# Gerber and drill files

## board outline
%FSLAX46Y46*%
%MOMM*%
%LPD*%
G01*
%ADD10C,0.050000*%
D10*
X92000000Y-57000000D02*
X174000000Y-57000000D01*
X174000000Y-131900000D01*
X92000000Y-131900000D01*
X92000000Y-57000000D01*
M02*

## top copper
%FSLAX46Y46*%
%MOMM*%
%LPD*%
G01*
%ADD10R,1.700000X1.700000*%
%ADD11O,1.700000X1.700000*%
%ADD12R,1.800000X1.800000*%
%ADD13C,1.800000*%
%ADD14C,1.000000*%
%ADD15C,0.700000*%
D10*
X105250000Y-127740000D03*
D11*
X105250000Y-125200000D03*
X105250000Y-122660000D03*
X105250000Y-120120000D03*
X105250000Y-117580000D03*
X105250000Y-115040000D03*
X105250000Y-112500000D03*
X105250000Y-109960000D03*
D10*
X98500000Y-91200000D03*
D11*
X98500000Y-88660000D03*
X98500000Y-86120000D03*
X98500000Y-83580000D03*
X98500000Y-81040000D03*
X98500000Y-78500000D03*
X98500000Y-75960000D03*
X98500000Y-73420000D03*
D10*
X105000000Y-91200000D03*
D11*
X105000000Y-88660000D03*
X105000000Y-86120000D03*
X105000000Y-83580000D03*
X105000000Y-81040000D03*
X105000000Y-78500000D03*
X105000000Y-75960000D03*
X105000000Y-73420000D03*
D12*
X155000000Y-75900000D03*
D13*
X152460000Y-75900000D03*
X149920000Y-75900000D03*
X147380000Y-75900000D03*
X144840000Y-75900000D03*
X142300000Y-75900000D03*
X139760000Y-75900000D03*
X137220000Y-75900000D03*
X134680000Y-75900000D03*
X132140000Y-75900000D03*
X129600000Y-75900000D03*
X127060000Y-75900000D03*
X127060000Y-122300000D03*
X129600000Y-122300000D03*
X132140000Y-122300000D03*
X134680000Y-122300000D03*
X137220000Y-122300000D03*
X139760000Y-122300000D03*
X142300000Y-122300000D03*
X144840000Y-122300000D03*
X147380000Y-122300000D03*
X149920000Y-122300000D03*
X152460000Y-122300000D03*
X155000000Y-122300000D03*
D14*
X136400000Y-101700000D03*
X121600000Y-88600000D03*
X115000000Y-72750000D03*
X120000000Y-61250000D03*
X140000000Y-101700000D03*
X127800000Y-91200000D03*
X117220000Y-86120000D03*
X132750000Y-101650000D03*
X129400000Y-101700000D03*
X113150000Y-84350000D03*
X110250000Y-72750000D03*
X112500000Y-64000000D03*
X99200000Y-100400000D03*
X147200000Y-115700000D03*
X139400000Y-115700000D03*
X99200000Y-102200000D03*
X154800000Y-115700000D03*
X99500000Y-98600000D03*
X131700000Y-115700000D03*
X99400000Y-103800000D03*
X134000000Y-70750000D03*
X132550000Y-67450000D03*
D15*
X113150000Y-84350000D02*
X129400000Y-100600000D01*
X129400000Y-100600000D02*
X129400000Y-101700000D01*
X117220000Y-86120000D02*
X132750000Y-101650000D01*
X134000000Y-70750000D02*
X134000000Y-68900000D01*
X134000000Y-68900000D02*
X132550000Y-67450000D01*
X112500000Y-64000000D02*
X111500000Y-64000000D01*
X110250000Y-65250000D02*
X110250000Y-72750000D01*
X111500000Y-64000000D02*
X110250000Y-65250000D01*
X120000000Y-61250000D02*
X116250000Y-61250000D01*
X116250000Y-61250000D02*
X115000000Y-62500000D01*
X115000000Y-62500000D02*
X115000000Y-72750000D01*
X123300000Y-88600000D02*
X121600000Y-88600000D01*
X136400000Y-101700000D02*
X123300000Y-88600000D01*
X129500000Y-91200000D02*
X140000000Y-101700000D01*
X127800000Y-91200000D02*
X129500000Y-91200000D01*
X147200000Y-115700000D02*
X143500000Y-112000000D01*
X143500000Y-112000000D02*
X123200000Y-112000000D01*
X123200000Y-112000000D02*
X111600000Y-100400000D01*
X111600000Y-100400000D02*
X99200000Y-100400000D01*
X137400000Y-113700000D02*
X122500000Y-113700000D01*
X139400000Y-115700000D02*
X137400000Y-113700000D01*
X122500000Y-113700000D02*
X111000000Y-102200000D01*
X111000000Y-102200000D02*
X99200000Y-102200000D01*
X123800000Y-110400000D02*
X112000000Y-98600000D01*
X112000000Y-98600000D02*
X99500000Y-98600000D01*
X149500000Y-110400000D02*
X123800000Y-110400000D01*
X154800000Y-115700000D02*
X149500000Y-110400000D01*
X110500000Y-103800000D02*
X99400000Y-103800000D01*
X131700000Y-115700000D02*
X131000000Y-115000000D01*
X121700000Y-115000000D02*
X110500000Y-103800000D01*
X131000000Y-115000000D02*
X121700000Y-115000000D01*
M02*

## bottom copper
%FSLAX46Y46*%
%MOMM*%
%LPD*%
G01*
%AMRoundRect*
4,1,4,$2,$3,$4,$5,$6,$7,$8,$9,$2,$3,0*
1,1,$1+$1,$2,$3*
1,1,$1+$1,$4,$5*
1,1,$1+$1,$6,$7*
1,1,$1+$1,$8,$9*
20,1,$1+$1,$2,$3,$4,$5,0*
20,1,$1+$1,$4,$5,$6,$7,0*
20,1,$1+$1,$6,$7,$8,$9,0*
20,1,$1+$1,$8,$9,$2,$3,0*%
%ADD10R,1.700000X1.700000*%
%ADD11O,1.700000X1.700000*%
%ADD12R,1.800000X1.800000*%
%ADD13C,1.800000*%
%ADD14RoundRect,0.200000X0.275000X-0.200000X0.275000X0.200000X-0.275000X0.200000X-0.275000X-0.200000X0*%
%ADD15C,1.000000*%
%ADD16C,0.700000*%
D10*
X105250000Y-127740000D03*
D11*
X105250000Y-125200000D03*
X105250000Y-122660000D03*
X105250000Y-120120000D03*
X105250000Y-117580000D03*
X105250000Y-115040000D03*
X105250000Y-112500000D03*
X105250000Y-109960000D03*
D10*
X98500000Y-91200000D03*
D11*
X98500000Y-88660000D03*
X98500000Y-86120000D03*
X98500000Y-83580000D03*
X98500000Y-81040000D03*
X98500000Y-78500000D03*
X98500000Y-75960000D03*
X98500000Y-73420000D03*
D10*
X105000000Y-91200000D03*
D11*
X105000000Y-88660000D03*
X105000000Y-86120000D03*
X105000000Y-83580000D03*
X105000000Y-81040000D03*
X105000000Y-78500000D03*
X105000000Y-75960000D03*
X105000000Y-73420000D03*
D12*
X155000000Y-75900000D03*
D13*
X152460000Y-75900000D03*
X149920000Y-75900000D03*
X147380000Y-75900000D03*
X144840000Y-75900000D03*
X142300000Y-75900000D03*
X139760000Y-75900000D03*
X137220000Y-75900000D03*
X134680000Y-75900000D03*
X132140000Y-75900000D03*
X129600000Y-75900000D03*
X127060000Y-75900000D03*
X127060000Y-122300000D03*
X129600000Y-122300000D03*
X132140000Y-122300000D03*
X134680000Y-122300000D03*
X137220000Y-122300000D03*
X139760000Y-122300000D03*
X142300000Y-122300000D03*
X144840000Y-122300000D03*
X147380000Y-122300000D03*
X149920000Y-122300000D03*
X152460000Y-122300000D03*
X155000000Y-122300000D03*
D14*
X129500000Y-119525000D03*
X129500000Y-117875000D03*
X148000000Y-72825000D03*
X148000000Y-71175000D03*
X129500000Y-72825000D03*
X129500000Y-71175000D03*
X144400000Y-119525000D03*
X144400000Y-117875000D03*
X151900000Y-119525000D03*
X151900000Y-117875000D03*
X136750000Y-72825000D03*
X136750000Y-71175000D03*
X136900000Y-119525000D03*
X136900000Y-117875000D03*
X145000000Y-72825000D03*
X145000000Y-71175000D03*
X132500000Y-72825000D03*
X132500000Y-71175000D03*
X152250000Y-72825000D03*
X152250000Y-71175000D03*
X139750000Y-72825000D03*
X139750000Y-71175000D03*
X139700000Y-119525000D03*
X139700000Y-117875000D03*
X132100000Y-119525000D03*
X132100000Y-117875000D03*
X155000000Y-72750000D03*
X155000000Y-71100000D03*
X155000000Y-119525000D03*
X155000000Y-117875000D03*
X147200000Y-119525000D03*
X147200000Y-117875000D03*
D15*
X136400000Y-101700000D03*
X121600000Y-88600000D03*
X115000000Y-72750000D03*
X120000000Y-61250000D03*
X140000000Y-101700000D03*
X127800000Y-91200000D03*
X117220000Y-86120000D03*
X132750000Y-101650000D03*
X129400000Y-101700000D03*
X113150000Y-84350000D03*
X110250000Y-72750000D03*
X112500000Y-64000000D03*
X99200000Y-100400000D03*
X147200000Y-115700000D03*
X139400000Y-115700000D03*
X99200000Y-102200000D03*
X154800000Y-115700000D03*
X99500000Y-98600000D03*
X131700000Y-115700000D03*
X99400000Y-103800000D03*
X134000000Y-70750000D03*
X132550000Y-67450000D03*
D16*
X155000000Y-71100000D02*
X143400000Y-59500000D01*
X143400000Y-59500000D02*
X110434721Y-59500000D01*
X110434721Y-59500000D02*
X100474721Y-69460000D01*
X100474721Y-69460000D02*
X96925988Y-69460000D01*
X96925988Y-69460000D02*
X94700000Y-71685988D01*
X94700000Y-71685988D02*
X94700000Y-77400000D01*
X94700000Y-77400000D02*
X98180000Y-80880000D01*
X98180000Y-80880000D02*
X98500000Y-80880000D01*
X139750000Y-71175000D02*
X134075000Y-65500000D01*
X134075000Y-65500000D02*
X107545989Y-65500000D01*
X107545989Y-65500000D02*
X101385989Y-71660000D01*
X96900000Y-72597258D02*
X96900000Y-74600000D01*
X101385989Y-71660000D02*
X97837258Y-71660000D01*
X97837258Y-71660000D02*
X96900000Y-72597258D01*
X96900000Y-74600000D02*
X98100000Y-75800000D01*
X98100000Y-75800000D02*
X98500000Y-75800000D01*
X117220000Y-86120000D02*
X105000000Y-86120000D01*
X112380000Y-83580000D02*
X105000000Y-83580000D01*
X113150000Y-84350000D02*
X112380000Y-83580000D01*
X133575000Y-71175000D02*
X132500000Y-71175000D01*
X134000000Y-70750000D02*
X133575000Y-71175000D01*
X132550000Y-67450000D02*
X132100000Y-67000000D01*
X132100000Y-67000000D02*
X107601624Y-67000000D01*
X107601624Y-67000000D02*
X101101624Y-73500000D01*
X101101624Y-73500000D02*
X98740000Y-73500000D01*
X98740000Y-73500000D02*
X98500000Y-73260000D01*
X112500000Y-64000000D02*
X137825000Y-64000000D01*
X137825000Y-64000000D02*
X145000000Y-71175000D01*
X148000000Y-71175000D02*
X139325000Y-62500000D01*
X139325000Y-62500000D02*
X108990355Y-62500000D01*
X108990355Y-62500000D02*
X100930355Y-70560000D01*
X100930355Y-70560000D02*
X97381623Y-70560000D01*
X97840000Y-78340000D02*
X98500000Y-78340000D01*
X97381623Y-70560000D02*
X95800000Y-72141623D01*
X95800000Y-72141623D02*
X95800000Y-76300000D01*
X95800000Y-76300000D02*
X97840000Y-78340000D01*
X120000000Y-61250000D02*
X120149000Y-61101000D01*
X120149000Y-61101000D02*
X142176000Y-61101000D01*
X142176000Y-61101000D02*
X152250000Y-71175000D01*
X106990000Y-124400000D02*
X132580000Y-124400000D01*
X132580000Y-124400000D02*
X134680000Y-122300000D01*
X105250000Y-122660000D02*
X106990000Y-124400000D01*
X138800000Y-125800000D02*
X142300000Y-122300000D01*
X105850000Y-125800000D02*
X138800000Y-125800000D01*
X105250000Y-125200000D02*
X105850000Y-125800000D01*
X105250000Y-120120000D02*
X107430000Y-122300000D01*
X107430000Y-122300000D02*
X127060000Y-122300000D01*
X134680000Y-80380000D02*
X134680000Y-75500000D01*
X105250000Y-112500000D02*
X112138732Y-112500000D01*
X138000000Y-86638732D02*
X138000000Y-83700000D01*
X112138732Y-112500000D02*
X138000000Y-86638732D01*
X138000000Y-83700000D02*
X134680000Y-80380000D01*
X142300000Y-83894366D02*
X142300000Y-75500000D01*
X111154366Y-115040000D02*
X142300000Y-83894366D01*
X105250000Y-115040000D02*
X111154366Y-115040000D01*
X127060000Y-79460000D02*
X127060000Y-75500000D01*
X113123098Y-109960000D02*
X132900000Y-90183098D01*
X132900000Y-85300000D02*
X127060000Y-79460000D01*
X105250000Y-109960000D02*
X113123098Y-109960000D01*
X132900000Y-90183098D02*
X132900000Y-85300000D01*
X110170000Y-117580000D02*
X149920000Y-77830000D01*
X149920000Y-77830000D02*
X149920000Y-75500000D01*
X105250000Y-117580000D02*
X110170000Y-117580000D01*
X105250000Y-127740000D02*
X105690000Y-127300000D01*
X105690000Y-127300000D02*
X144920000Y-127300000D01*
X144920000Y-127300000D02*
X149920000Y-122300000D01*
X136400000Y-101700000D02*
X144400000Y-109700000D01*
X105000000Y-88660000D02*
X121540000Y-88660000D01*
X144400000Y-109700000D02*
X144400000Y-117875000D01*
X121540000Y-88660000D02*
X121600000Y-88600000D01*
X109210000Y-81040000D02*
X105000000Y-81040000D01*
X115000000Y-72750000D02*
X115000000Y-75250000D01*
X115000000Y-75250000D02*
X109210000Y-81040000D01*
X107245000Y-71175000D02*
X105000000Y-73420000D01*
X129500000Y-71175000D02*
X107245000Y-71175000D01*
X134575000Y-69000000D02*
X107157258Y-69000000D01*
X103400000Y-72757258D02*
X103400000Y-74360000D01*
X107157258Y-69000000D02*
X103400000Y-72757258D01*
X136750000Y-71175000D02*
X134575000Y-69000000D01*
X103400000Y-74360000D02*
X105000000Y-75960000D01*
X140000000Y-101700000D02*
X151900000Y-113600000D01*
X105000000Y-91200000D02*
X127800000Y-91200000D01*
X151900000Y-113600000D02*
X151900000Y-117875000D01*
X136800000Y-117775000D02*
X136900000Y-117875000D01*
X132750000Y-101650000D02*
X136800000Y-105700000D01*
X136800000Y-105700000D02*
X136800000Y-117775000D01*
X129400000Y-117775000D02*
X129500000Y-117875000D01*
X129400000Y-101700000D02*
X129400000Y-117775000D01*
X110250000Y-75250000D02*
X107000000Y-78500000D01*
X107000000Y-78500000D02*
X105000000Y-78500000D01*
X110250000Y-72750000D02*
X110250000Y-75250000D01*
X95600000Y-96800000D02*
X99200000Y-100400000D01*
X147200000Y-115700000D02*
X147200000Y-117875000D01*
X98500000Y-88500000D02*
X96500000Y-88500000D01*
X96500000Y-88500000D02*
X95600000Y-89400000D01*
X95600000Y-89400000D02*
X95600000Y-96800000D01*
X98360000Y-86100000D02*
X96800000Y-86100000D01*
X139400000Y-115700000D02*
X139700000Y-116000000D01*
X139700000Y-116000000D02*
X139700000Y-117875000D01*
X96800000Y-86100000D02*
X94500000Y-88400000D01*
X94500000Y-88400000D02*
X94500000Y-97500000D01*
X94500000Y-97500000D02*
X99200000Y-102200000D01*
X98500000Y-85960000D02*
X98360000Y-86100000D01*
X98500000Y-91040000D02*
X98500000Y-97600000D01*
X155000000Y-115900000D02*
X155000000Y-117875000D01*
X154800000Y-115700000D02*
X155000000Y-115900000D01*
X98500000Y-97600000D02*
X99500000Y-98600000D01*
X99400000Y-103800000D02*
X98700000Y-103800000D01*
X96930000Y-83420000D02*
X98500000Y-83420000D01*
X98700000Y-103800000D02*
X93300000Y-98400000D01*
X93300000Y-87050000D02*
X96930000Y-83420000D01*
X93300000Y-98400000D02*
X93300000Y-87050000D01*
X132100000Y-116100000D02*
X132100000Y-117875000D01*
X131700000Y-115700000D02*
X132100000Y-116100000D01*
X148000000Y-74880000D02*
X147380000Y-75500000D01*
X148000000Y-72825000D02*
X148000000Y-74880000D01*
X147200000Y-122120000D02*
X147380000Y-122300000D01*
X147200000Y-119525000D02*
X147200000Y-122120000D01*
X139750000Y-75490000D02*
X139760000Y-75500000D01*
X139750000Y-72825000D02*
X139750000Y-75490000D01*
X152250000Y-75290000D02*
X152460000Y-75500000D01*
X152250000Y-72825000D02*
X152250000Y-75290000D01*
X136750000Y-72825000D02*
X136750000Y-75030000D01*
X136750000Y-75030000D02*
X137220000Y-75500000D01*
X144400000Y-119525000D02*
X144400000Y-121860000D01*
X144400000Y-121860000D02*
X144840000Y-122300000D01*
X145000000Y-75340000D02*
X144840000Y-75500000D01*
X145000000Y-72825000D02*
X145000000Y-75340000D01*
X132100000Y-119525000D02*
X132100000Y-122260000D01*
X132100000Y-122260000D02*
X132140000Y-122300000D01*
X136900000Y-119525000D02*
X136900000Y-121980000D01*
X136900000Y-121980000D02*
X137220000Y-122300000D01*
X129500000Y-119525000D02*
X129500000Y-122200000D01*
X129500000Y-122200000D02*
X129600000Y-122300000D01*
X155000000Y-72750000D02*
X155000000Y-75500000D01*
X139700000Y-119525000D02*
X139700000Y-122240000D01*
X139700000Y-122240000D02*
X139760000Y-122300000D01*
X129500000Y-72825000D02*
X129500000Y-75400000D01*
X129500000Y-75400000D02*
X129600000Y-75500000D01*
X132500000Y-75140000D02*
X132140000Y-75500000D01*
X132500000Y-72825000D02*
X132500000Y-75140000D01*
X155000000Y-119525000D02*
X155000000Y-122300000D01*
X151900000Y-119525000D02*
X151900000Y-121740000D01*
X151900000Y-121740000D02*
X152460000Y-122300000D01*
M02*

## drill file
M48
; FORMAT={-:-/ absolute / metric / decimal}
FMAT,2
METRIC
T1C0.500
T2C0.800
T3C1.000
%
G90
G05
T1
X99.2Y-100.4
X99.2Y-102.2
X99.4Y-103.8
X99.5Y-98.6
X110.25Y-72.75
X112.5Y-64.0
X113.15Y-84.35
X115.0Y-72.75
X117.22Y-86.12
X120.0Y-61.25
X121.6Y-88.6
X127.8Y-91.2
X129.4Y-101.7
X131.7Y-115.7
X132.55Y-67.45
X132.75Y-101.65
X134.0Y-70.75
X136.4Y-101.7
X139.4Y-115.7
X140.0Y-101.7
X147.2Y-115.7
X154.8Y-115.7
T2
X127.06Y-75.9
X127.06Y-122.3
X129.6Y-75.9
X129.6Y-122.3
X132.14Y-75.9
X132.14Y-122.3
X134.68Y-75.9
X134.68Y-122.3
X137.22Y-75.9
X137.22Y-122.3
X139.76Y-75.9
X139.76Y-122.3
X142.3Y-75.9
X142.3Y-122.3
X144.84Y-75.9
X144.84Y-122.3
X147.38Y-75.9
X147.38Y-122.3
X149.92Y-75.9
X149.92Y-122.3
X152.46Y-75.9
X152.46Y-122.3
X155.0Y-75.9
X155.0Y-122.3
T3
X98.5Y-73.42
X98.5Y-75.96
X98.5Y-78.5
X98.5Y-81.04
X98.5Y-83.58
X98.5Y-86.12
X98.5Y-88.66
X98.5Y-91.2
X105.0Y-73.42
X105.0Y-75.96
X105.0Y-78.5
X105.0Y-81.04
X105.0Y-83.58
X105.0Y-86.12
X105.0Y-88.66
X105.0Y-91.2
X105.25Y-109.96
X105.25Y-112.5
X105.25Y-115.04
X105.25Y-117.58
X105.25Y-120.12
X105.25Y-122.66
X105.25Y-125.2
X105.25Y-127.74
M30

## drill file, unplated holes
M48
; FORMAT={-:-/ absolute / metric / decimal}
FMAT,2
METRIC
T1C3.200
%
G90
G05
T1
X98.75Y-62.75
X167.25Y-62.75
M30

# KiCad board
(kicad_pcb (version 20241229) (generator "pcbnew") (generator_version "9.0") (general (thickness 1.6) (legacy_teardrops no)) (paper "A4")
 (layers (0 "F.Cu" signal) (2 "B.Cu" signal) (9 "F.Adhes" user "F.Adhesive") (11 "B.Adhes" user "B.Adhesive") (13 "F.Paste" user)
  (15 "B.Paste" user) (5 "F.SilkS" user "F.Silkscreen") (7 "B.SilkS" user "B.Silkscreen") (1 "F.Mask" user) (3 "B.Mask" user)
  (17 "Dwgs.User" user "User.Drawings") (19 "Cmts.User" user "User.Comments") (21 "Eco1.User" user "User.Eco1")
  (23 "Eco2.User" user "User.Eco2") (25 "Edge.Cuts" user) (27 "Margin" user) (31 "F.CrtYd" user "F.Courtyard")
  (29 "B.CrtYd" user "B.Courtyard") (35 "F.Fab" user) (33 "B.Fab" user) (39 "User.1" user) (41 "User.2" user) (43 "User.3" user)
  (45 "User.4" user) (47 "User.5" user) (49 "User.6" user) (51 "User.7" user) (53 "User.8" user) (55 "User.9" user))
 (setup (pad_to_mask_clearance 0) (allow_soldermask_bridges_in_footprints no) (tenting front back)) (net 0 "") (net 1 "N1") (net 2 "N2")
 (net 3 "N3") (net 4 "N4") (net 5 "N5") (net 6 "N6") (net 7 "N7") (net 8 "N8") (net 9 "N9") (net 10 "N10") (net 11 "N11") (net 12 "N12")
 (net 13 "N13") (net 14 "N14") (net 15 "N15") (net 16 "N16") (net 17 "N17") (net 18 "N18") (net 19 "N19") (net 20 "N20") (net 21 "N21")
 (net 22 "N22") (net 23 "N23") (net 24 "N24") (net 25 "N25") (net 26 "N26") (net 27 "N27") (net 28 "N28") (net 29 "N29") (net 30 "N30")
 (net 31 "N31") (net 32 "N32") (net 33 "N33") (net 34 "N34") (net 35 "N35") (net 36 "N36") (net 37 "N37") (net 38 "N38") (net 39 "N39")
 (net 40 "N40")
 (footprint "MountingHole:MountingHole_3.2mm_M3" (layer "F.Cu") (at 98.75 62.75)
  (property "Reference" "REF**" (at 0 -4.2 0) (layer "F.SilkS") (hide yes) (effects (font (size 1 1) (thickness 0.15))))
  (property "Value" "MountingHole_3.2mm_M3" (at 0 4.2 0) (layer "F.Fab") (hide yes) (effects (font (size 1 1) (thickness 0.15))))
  (pad "" np_thru_hole circle (at 0 0) (size 3.2 3.2) (drill 3.2) (layers "*.Cu" "*.Mask")))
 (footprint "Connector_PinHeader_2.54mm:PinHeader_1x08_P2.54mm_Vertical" (layer "F.Cu") (at 105.25 127.74 180)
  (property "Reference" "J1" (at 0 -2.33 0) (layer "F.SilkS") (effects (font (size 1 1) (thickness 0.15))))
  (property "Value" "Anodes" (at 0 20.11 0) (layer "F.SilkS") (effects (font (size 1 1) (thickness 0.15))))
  (pad "1" thru_hole rect (at 0 0 180) (size 1.7 1.7) (drill 1) (layers "*.Cu" "*.Mask") (remove_unused_layers no) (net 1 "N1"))
  (pad "2" thru_hole oval (at 0 2.54 180) (size 1.7 1.7) (drill 1) (layers "*.Cu" "*.Mask") (remove_unused_layers no) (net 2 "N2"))
  (pad "3" thru_hole oval (at 0 5.08 180) (size 1.7 1.7) (drill 1) (layers "*.Cu" "*.Mask") (remove_unused_layers no) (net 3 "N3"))
  (pad "4" thru_hole oval (at 0 7.62 180) (size 1.7 1.7) (drill 1) (layers "*.Cu" "*.Mask") (remove_unused_layers no) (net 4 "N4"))
  (pad "5" thru_hole oval (at 0 10.16 180) (size 1.7 1.7) (drill 1) (layers "*.Cu" "*.Mask") (remove_unused_layers no) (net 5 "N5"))
  (pad "6" thru_hole oval (at 0 12.7 180) (size 1.7 1.7) (drill 1) (layers "*.Cu" "*.Mask") (remove_unused_layers no) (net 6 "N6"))
  (pad "7" thru_hole oval (at 0 15.24 180) (size 1.7 1.7) (drill 1) (layers "*.Cu" "*.Mask") (remove_unused_layers no) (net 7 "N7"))
  (pad "8" thru_hole oval (at 0 17.78 180) (size 1.7 1.7) (drill 1) (layers "*.Cu" "*.Mask") (remove_unused_layers no) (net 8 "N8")))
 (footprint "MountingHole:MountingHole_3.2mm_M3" (layer "F.Cu") (at 167.25 62.75)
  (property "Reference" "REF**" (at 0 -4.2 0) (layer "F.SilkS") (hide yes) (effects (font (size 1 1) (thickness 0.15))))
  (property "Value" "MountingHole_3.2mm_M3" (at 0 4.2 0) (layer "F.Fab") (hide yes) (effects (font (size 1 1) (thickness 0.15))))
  (pad "" np_thru_hole circle (at 0 0) (size 3.2 3.2) (drill 3.2) (layers "*.Cu" "*.Mask")))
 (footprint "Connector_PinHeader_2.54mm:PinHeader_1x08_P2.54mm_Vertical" (layer "F.Cu") (at 98.5 91.2 180)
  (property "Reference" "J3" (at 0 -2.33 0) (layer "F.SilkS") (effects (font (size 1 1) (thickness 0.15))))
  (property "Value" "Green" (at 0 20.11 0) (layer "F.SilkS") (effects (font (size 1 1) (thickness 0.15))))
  (pad "1" thru_hole rect (at 0 0 180) (size 1.7 1.7) (drill 1) (layers "*.Cu" "*.Mask") (remove_unused_layers no) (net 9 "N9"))
  (pad "2" thru_hole oval (at 0 2.54 180) (size 1.7 1.7) (drill 1) (layers "*.Cu" "*.Mask") (remove_unused_layers no) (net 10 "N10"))
  (pad "3" thru_hole oval (at 0 5.08 180) (size 1.7 1.7) (drill 1) (layers "*.Cu" "*.Mask") (remove_unused_layers no) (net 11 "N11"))
  (pad "4" thru_hole oval (at 0 7.62 180) (size 1.7 1.7) (drill 1) (layers "*.Cu" "*.Mask") (remove_unused_layers no) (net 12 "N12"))
  (pad "5" thru_hole oval (at 0 10.16 180) (size 1.7 1.7) (drill 1) (layers "*.Cu" "*.Mask") (remove_unused_layers no) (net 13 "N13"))
  (pad "6" thru_hole oval (at 0 12.7 180) (size 1.7 1.7) (drill 1) (layers "*.Cu" "*.Mask") (remove_unused_layers no) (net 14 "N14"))
  (pad "7" thru_hole oval (at 0 15.24 180) (size 1.7 1.7) (drill 1) (layers "*.Cu" "*.Mask") (remove_unused_layers no) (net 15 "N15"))
  (pad "8" thru_hole oval (at 0 17.78 180) (size 1.7 1.7) (drill 1) (layers "*.Cu" "*.Mask") (remove_unused_layers no) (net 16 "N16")))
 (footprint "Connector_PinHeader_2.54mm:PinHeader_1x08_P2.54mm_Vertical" (layer "F.Cu") (at 105 91.2 180)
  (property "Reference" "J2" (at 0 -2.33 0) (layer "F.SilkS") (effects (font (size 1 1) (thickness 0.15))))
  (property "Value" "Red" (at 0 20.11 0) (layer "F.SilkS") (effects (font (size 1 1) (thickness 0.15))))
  (pad "1" thru_hole rect (at 0 0 180) (size 1.7 1.7) (drill 1) (layers "*.Cu" "*.Mask") (remove_unused_layers no) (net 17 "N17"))
  (pad "2" thru_hole oval (at 0 2.54 180) (size 1.7 1.7) (drill 1) (layers "*.Cu" "*.Mask") (remove_unused_layers no) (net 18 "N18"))
  (pad "3" thru_hole oval (at 0 5.08 180) (size 1.7 1.7) (drill 1) (layers "*.Cu" "*.Mask") (remove_unused_layers no) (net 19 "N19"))
  (pad "4" thru_hole oval (at 0 7.62 180) (size 1.7 1.7) (drill 1) (layers "*.Cu" "*.Mask") (remove_unused_layers no) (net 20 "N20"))
  (pad "5" thru_hole oval (at 0 10.16 180) (size 1.7 1.7) (drill 1) (layers "*.Cu" "*.Mask") (remove_unused_layers no) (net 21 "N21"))
  (pad "6" thru_hole oval (at 0 12.7 180) (size 1.7 1.7) (drill 1) (layers "*.Cu" "*.Mask") (remove_unused_layers no) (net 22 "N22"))
  (pad "7" thru_hole oval (at 0 15.24 180) (size 1.7 1.7) (drill 1) (layers "*.Cu" "*.Mask") (remove_unused_layers no) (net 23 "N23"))
  (pad "8" thru_hole oval (at 0 17.78 180) (size 1.7 1.7) (drill 1) (layers "*.Cu" "*.Mask") (remove_unused_layers no) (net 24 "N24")))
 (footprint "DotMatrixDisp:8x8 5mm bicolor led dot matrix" (layer "F.Cu") (at 112 70.1)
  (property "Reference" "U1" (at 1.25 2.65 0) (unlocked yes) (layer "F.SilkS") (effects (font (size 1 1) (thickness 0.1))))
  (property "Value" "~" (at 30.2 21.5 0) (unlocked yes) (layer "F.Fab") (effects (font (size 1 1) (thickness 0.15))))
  (pad "1" thru_hole rect (at 43 5.8) (size 1.8 1.8) (drill 0.8) (layers "*.Cu" "*.Mask") (remove_unused_layers no) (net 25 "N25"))
  (pad "2" thru_hole circle (at 40.46 5.8) (size 1.8 1.8) (drill 0.8) (layers "*.Cu" "*.Mask") (remove_unused_layers no) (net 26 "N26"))
  (pad "3" thru_hole circle (at 37.92 5.8) (size 1.8 1.8) (drill 0.8) (layers "*.Cu" "*.Mask") (remove_unused_layers no) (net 5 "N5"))
  (pad "4" thru_hole circle (at 35.38 5.8) (size 1.8 1.8) (drill 0.8) (layers "*.Cu" "*.Mask") (remove_unused_layers no) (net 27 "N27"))
  (pad "5" thru_hole circle (at 32.84 5.8) (size 1.8 1.8) (drill 0.8) (layers "*.Cu" "*.Mask") (remove_unused_layers no) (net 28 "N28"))
  (pad "6" thru_hole circle (at 30.3 5.8) (size 1.8 1.8) (drill 0.8) (layers "*.Cu" "*.Mask") (remove_unused_layers no) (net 6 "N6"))
  (pad "7" thru_hole circle (at 27.76 5.8) (size 1.8 1.8) (drill 0.8) (layers "*.Cu" "*.Mask") (remove_unused_layers no) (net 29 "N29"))
  (pad "8" thru_hole circle (at 25.22 5.8) (size 1.8 1.8) (drill 0.8) (layers "*.Cu" "*.Mask") (remove_unused_layers no) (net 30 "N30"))
  (pad "9" thru_hole circle (at 22.68 5.8) (size 1.8 1.8) (drill 0.8) (layers "*.Cu" "*.Mask") (remove_unused_layers no) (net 7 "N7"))
  (pad "10" thru_hole circle (at 20.14 5.8) (size 1.8 1.8) (drill 0.8) (layers "*.Cu" "*.Mask") (remove_unused_layers no) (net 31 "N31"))
  (pad "11" thru_hole circle (at 17.6 5.8) (size 1.8 1.8) (drill 0.8) (layers "*.Cu" "*.Mask") (remove_unused_layers no) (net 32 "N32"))
  (pad "12" thru_hole circle (at 15.06 5.8) (size 1.8 1.8) (drill 0.8) (layers "*.Cu" "*.Mask") (remove_unused_layers no) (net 8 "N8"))
  (pad "13" thru_hole circle (at 15.06 52.2) (size 1.8 1.8) (drill 0.8) (layers "*.Cu" "*.Mask") (remove_unused_layers no) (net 4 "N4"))
  (pad "14" thru_hole circle (at 17.6 52.2) (size 1.8 1.8) (drill 0.8) (layers "*.Cu" "*.Mask") (remove_unused_layers no) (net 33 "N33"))
  (pad "15" thru_hole circle (at 20.14 52.2) (size 1.8 1.8) (drill 0.8) (layers "*.Cu" "*.Mask") (remove_unused_layers no) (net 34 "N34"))
  (pad "16" thru_hole circle (at 22.68 52.2) (size 1.8 1.8) (drill 0.8) (layers "*.Cu" "*.Mask") (remove_unused_layers no) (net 3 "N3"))
  (pad "17" thru_hole circle (at 25.22 52.2) (size 1.8 1.8) (drill 0.8) (layers "*.Cu" "*.Mask") (remove_unused_layers no) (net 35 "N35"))
  (pad "18" thru_hole circle (at 27.76 52.2) (size 1.8 1.8) (drill 0.8) (layers "*.Cu" "*.Mask") (remove_unused_layers no) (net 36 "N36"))
  (pad "19" thru_hole circle (at 30.3 52.2) (size 1.8 1.8) (drill 0.8) (layers "*.Cu" "*.Mask") (remove_unused_layers no) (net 2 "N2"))
  (pad "20" thru_hole circle (at 32.84 52.2) (size 1.8 1.8) (drill 0.8) (layers "*.Cu" "*.Mask") (remove_unused_layers no) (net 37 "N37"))
  (pad "21" thru_hole circle (at 35.38 52.2) (size 1.8 1.8) (drill 0.8) (layers "*.Cu" "*.Mask") (remove_unused_layers no) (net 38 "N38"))
  (pad "22" thru_hole circle (at 37.92 52.2) (size 1.8 1.8) (drill 0.8) (layers "*.Cu" "*.Mask") (remove_unused_layers no) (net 1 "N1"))
  (pad "23" thru_hole circle (at 40.46 52.2) (size 1.8 1.8) (drill 0.8) (layers "*.Cu" "*.Mask") (remove_unused_layers no) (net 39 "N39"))
  (pad "24" thru_hole circle (at 43 52.2) (size 1.8 1.8) (drill 0.8) (layers "*.Cu" "*.Mask") (remove_unused_layers no) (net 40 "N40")))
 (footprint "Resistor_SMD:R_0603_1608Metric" (layer "B.Cu") (at 129.5 118.7 90)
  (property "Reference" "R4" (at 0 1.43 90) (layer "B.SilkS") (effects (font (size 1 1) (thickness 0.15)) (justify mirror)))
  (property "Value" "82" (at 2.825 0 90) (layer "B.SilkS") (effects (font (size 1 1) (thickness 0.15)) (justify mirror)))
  (pad "1" smd roundrect (at -0.825 0 90) (size 0.8 0.95) (layers "B.Cu" "B.Mask" "B.Paste") (roundrect_rratio 0.25) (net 33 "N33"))
  (pad "2" smd roundrect (at 0.825 0 90) (size 0.8 0.95) (layers "B.Cu" "B.Mask" "B.Paste") (roundrect_rratio 0.25) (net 20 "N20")))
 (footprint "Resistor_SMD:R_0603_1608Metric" (layer "B.Cu") (at 148 72 90)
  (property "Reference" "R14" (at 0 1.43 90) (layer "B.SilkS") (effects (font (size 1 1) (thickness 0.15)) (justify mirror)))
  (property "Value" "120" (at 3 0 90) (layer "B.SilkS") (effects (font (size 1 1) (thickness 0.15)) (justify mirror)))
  (pad "1" smd roundrect (at -0.825 0 90) (size 0.8 0.95) (layers "B.Cu" "B.Mask" "B.Paste") (roundrect_rratio 0.25) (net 27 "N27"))
  (pad "2" smd roundrect (at 0.825 0 90) (size 0.8 0.95) (layers "B.Cu" "B.Mask" "B.Paste") (roundrect_rratio 0.25) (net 14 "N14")))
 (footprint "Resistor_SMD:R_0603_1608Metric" (layer "B.Cu") (at 129.5 72 90)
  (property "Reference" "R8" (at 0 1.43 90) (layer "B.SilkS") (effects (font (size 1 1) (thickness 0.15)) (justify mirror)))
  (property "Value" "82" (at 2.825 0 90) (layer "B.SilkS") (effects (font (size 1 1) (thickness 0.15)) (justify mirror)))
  (pad "1" smd roundrect (at -0.825 0 90) (size 0.8 0.95) (layers "B.Cu" "B.Mask" "B.Paste") (roundrect_rratio 0.25) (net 32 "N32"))
  (pad "2" smd roundrect (at 0.825 0 90) (size 0.8 0.95) (layers "B.Cu" "B.Mask" "B.Paste") (roundrect_rratio 0.25) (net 24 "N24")))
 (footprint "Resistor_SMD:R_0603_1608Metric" (layer "B.Cu") (at 144.4 118.7 90)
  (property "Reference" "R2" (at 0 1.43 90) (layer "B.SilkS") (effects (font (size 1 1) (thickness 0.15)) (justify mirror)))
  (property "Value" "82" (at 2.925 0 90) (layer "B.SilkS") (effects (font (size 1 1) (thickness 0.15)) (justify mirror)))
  (pad "1" smd roundrect (at -0.825 0 90) (size 0.8 0.95) (layers "B.Cu" "B.Mask" "B.Paste") (roundrect_rratio 0.25) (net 37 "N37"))
  (pad "2" smd roundrect (at 0.825 0 90) (size 0.8 0.95) (layers "B.Cu" "B.Mask" "B.Paste") (roundrect_rratio 0.25) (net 18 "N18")))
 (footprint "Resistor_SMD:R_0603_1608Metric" (layer "B.Cu") (at 151.9 118.7 90)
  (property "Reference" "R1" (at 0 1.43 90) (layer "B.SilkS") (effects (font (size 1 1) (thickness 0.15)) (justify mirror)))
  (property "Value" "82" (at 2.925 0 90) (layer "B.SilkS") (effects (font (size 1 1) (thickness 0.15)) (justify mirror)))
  (pad "1" smd roundrect (at -0.825 0 90) (size 0.8 0.95) (layers "B.Cu" "B.Mask" "B.Paste") (roundrect_rratio 0.25) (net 39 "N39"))
  (pad "2" smd roundrect (at 0.825 0 90) (size 0.8 0.95) (layers "B.Cu" "B.Mask" "B.Paste") (roundrect_rratio 0.25) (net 17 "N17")))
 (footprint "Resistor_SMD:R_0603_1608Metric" (layer "B.Cu") (at 136.75 72 90)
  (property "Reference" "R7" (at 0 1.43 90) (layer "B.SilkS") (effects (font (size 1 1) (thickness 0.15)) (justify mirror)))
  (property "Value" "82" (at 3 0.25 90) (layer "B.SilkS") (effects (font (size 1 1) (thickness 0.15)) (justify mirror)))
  (pad "1" smd roundrect (at -0.825 0 90) (size 0.8 0.95) (layers "B.Cu" "B.Mask" "B.Paste") (roundrect_rratio 0.25) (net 30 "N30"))
  (pad "2" smd roundrect (at 0.825 0 90) (size 0.8 0.95) (layers "B.Cu" "B.Mask" "B.Paste") (roundrect_rratio 0.25) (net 23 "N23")))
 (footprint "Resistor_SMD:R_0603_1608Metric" (layer "B.Cu") (at 136.9 118.7 90)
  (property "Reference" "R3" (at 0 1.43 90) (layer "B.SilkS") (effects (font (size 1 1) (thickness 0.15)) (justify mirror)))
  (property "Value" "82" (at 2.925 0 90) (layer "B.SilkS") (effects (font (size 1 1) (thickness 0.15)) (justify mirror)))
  (pad "1" smd roundrect (at -0.825 0 90) (size 0.8 0.95) (layers "B.Cu" "B.Mask" "B.Paste") (roundrect_rratio 0.25) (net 35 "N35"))
  (pad "2" smd roundrect (at 0.825 0 90) (size 0.8 0.95) (layers "B.Cu" "B.Mask" "B.Paste") (roundrect_rratio 0.25) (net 19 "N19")))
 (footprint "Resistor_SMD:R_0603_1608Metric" (layer "B.Cu") (at 145 72 90)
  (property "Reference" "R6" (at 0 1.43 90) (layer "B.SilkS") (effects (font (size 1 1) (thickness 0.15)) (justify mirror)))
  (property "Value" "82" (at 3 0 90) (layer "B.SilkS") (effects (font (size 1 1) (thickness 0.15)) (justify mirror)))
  (pad "1" smd roundrect (at -0.825 0 90) (size 0.8 0.95) (layers "B.Cu" "B.Mask" "B.Paste") (roundrect_rratio 0.25) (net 28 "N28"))
  (pad "2" smd roundrect (at 0.825 0 90) (size 0.8 0.95) (layers "B.Cu" "B.Mask" "B.Paste") (roundrect_rratio 0.25) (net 22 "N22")))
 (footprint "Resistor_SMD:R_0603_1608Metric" (layer "B.Cu") (at 132.5 72 90)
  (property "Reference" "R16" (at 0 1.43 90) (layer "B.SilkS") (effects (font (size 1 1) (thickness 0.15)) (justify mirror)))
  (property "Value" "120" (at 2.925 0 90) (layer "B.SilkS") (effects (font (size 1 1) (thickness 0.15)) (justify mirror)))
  (pad "1" smd roundrect (at -0.825 0 90) (size 0.8 0.95) (layers "B.Cu" "B.Mask" "B.Paste") (roundrect_rratio 0.25) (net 31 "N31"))
  (pad "2" smd roundrect (at 0.825 0 90) (size 0.8 0.95) (layers "B.Cu" "B.Mask" "B.Paste") (roundrect_rratio 0.25) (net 16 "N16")))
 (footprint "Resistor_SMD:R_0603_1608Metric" (layer "B.Cu") (at 152.25 72 90)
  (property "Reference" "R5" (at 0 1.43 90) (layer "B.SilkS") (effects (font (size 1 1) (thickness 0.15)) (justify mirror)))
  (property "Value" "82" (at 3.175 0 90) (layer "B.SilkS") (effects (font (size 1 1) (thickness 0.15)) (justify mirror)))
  (pad "1" smd roundrect (at -0.825 0 90) (size 0.8 0.95) (layers "B.Cu" "B.Mask" "B.Paste") (roundrect_rratio 0.25) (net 26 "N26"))
  (pad "2" smd roundrect (at 0.825 0 90) (size 0.8 0.95) (layers "B.Cu" "B.Mask" "B.Paste") (roundrect_rratio 0.25) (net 21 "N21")))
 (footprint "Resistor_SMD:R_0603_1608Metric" (layer "B.Cu") (at 139.75 72 90)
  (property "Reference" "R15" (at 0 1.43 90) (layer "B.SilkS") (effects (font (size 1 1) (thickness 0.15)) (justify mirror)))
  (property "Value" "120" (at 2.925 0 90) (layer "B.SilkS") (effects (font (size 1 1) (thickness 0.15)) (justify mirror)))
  (pad "1" smd roundrect (at -0.825 0 90) (size 0.8 0.95) (layers "B.Cu" "B.Mask" "B.Paste") (roundrect_rratio 0.25) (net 29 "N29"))
  (pad "2" smd roundrect (at 0.825 0 90) (size 0.8 0.95) (layers "B.Cu" "B.Mask" "B.Paste") (roundrect_rratio 0.25) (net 15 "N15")))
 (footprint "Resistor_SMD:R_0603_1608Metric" (layer "B.Cu") (at 139.7 118.7 90)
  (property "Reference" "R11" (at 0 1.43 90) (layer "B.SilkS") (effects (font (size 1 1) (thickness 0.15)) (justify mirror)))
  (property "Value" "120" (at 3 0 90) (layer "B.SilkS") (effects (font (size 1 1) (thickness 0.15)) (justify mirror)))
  (pad "1" smd roundrect (at -0.825 0 90) (size 0.8 0.95) (layers "B.Cu" "B.Mask" "B.Paste") (roundrect_rratio 0.25) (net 36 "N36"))
  (pad "2" smd roundrect (at 0.825 0 90) (size 0.8 0.95) (layers "B.Cu" "B.Mask" "B.Paste") (roundrect_rratio 0.25) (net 11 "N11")))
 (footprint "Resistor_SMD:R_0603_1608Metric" (layer "B.Cu") (at 132.1 118.7 90)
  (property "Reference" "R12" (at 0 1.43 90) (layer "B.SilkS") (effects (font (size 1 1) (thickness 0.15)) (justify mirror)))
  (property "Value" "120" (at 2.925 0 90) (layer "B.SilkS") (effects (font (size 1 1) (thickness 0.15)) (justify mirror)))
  (pad "1" smd roundrect (at -0.825 0 90) (size 0.8 0.95) (layers "B.Cu" "B.Mask" "B.Paste") (roundrect_rratio 0.25) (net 34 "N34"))
  (pad "2" smd roundrect (at 0.825 0 90) (size 0.8 0.95) (layers "B.Cu" "B.Mask" "B.Paste") (roundrect_rratio 0.25) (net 12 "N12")))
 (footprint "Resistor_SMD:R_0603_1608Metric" (layer "B.Cu") (at 155 71.925 90)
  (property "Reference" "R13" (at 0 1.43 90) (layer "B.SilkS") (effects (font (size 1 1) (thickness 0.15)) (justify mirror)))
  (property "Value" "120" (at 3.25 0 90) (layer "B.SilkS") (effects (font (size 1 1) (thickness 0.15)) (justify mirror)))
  (pad "1" smd roundrect (at -0.825 0 90) (size 0.8 0.95) (layers "B.Cu" "B.Mask" "B.Paste") (roundrect_rratio 0.25) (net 25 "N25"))
  (pad "2" smd roundrect (at 0.825 0 90) (size 0.8 0.95) (layers "B.Cu" "B.Mask" "B.Paste") (roundrect_rratio 0.25) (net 13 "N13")))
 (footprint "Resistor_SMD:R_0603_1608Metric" (layer "B.Cu") (at 155 118.7 90)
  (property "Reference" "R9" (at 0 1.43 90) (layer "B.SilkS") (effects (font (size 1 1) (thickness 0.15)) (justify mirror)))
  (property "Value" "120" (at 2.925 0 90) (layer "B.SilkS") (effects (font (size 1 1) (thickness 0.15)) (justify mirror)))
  (pad "1" smd roundrect (at -0.825 0 90) (size 0.8 0.95) (layers "B.Cu" "B.Mask" "B.Paste") (roundrect_rratio 0.25) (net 40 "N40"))
  (pad "2" smd roundrect (at 0.825 0 90) (size 0.8 0.95) (layers "B.Cu" "B.Mask" "B.Paste") (roundrect_rratio 0.25) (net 9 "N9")))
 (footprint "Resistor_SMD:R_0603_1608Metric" (layer "B.Cu") (at 147.2 118.7 90)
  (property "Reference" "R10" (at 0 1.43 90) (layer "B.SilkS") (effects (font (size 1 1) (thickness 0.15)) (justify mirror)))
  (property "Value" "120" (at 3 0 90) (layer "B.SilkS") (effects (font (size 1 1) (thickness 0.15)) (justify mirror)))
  (pad "1" smd roundrect (at -0.825 0 90) (size 0.8 0.95) (layers "B.Cu" "B.Mask" "B.Paste") (roundrect_rratio 0.25) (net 38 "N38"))
  (pad "2" smd roundrect (at 0.825 0 90) (size 0.8 0.95) (layers "B.Cu" "B.Mask" "B.Paste") (roundrect_rratio 0.25) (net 10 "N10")))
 (gr_rect (start 92 57) (end 174 131.9) (stroke (width 0.05) (type default)) (fill no) (layer "Edge.Cuts"))
 (segment (start 106.99 124.4) (end 132.58 124.4) (width 0.7) (layer "B.Cu") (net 3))
 (segment (start 132.58 124.4) (end 134.68 122.3) (width 0.7) (layer "B.Cu") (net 3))
 (segment (start 105.25 122.66) (end 106.99 124.4) (width 0.7) (layer "B.Cu") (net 3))
 (segment (start 138.8 125.8) (end 142.3 122.3) (width 0.7) (layer "B.Cu") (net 2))
 (segment (start 105.85 125.8) (end 138.8 125.8) (width 0.7) (layer "B.Cu") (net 2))
 (segment (start 105.25 125.2) (end 105.85 125.8) (width 0.7) (layer "B.Cu") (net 2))
 (segment (start 105.25 120.12) (end 107.43 122.3) (width 0.7) (layer "B.Cu") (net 4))
 (segment (start 107.43 122.3) (end 127.06 122.3) (width 0.7) (layer "B.Cu") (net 4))
 (segment (start 134.68 80.38) (end 134.68 75.5) (width 0.7) (layer "B.Cu") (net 7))
 (segment (start 105.25 112.5) (end 112.138732 112.5) (width 0.7) (layer "B.Cu") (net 7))
 (segment (start 138 86.638732) (end 138 83.7) (width 0.7) (layer "B.Cu") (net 7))
 (segment (start 112.138732 112.5) (end 138 86.638732) (width 0.7) (layer "B.Cu") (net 7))
 (segment (start 138 83.7) (end 134.68 80.38) (width 0.7) (layer "B.Cu") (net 7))
 (segment (start 142.3 83.894366) (end 142.3 75.5) (width 0.7) (layer "B.Cu") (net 6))
 (segment (start 111.154366 115.04) (end 142.3 83.894366) (width 0.7) (layer "B.Cu") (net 6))
 (segment (start 105.25 115.04) (end 111.154366 115.04) (width 0.7) (layer "B.Cu") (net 6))
 (segment (start 127.06 79.46) (end 127.06 75.5) (width 0.7) (layer "B.Cu") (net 8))
 (segment (start 113.123098 109.96) (end 132.9 90.183098) (width 0.7) (layer "B.Cu") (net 8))
 (segment (start 132.9 85.3) (end 127.06 79.46) (width 0.7) (layer "B.Cu") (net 8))
 (segment (start 105.25 109.96) (end 113.123098 109.96) (width 0.7) (layer "B.Cu") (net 8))
 (segment (start 132.9 90.183098) (end 132.9 85.3) (width 0.7) (layer "B.Cu") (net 8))
 (segment (start 110.17 117.58) (end 149.92 77.83) (width 0.7) (layer "B.Cu") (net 5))
 (segment (start 149.92 77.83) (end 149.92 75.5) (width 0.7) (layer "B.Cu") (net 5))
 (segment (start 105.25 117.58) (end 110.17 117.58) (width 0.7) (layer "B.Cu") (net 5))
 (segment (start 105.25 127.74) (end 105.69 127.3) (width 0.7) (layer "B.Cu") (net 1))
 (segment (start 105.69 127.3) (end 144.92 127.3) (width 0.7) (layer "B.Cu") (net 1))
 (segment (start 144.92 127.3) (end 149.92 122.3) (width 0.7) (layer "B.Cu") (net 1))
 (segment (start 123.3 88.6) (end 121.6 88.6) (width 0.7) (layer "F.Cu") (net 18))
 (segment (start 136.4 101.7) (end 123.3 88.6) (width 0.7) (layer "F.Cu") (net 18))
 (via (at 136.4 101.7) (size 1) (drill 0.5) (layers "F.Cu" "B.Cu") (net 18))
 (via (at 121.6 88.6) (size 1) (drill 0.5) (layers "F.Cu" "B.Cu") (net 18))
 (segment (start 136.4 101.7) (end 144.4 109.7) (width 0.7) (layer "B.Cu") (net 18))
 (segment (start 105 88.66) (end 121.54 88.66) (width 0.7) (layer "B.Cu") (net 18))
 (segment (start 144.4 109.7) (end 144.4 117.875) (width 0.7) (layer "B.Cu") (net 18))
 (segment (start 121.54 88.66) (end 121.6 88.6) (width 0.7) (layer "B.Cu") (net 18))
 (segment (start 120 61.25) (end 116.25 61.25) (width 0.7) (layer "F.Cu") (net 21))
 (segment (start 115 62.5) (end 115 72.75) (width 0.7) (layer "F.Cu") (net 21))
 (segment (start 116.25 61.25) (end 115 62.5) (width 0.7) (layer "F.Cu") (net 21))
 (via (at 115 72.75) (size 1) (drill 0.5) (layers "F.Cu" "B.Cu") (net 21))
 (via (at 120 61.25) (size 1) (drill 0.5) (layers "F.Cu" "B.Cu") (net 21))
 (segment (start 120.149 61.101) (end 142.176 61.101) (width 0.7) (layer "B.Cu") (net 21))
 (segment (start 109.21 81.04) (end 105 81.04) (width 0.7) (layer "B.Cu") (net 21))
 (segment (start 115 72.75) (end 115 75.25) (width 0.7) (layer "B.Cu") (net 21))
 (segment (start 142.176 61.101) (end 152.25 71.175) (width 0.7) (layer "B.Cu") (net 21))
 (segment (start 115 75.25) (end 109.21 81.04) (width 0.7) (layer "B.Cu") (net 21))
 (segment (start 120 61.25) (end 120.149 61.101) (width 0.7) (layer "B.Cu") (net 21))
 (segment (start 107.245 71.175) (end 105 73.42) (width 0.7) (layer "B.Cu") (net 24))
 (segment (start 129.5 71.175) (end 107.245 71.175) (width 0.7) (layer "B.Cu") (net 24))
 (segment (start 134.575 69) (end 107.157258 69) (width 0.7) (layer "B.Cu") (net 23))
 (segment (start 103.4 72.757258) (end 103.4 74.36) (width 0.7) (layer "B.Cu") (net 23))
 (segment (start 107.157258 69) (end 103.4 72.757258) (width 0.7) (layer "B.Cu") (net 23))
 (segment (start 136.75 71.175) (end 134.575 69) (width 0.7) (layer "B.Cu") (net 23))
 (segment (start 103.4 74.36) (end 105 75.96) (width 0.7) (layer "B.Cu") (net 23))
 (segment (start 129.5 91.2) (end 140 101.7) (width 0.7) (layer "F.Cu") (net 17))
 (segment (start 127.8 91.2) (end 129.5 91.2) (width 0.7) (layer "F.Cu") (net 17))
 (via (at 140 101.7) (size 1) (drill 0.5) (layers "F.Cu" "B.Cu") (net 17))
 (via (at 127.8 91.2) (size 1) (drill 0.5) (layers "F.Cu" "B.Cu") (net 17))
 (segment (start 140 101.7) (end 151.9 113.6) (width 0.7) (layer "B.Cu") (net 17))
 (segment (start 105 91.2) (end 127.8 91.2) (width 0.7) (layer "B.Cu") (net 17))
 (segment (start 151.9 113.6) (end 151.9 117.875) (width 0.7) (layer "B.Cu") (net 17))
 (segment (start 117.22 86.12) (end 132.75 101.65) (width 0.7) (layer "F.Cu") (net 19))
 (via (at 117.22 86.12) (size 1) (drill 0.5) (layers "F.Cu" "B.Cu") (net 19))
 (via (at 132.75 101.65) (size 1) (drill 0.5) (layers "F.Cu" "B.Cu") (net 19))
 (segment (start 136.8 117.775) (end 136.9 117.875) (width 0.7) (layer "B.Cu") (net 19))
 (segment (start 117.22 86.12) (end 105 86.12) (width 0.7) (layer "B.Cu") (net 19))
 (segment (start 132.75 101.65) (end 136.8 105.7) (width 0.7) (layer "B.Cu") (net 19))
 (segment (start 136.8 105.7) (end 136.8 117.775) (width 0.7) (layer "B.Cu") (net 19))
 (segment (start 113.15 84.35) (end 129.4 100.6) (width 0.7) (layer "F.Cu") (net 20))
 (segment (start 129.4 100.6) (end 129.4 101.7) (width 0.7) (layer "F.Cu") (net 20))
 (via (at 129.4 101.7) (size 1) (drill 0.5) (layers "F.Cu" "B.Cu") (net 20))
 (via (at 113.15 84.35) (size 1) (drill 0.5) (layers "F.Cu" "B.Cu") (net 20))
 (segment (start 112.38 83.58) (end 105 83.58) (width 0.7) (layer "B.Cu") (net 20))
 (segment (start 129.4 117.775) (end 129.5 117.875) (width 0.7) (layer "B.Cu") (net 20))
 (segment (start 113.15 84.35) (end 112.38 83.58) (width 0.7) (layer "B.Cu") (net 20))
 (segment (start 129.4 101.7) (end 129.4 117.775) (width 0.7) (layer "B.Cu") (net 20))
 (segment (start 112.5 64) (end 111.5 64) (width 0.7) (layer "F.Cu") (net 22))
 (segment (start 110.25 65.25) (end 110.25 72.75) (width 0.7) (layer "F.Cu") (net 22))
 (segment (start 111.5 64) (end 110.25 65.25) (width 0.7) (layer "F.Cu") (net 22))
 (via (at 110.25 72.75) (size 1) (drill 0.5) (layers "F.Cu" "B.Cu") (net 22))
 (via (at 112.5 64) (size 1) (drill 0.5) (layers "F.Cu" "B.Cu") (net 22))
 (segment (start 110.25 75.25) (end 107 78.5) (width 0.7) (layer "B.Cu") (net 22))
 (segment (start 137.825 64) (end 145 71.175) (width 0.7) (layer "B.Cu") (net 22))
 (segment (start 112.5 64) (end 137.825 64) (width 0.7) (layer "B.Cu") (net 22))
 (segment (start 107 78.5) (end 105 78.5) (width 0.7) (layer "B.Cu") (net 22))
 (segment (start 110.25 72.75) (end 110.25 75.25) (width 0.7) (layer "B.Cu") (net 22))
 (segment (start 96.9 72.597258) (end 96.9 74.6) (width 0.7) (layer "B.Cu") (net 15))
 (segment (start 101.385989 71.66) (end 97.837258 71.66) (width 0.7) (layer "B.Cu") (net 15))
 (segment (start 107.545989 65.5) (end 101.385989 71.66) (width 0.7) (layer "B.Cu") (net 15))
 (segment (start 98.1 75.8) (end 98.5 75.8) (width 0.7) (layer "B.Cu") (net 15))
 (segment (start 96.9 74.6) (end 98.1 75.8) (width 0.7) (layer "B.Cu") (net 15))
 (segment (start 97.837258 71.66) (end 96.9 72.597258) (width 0.7) (layer "B.Cu") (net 15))
 (segment (start 139.75 71.175) (end 134.075 65.5) (width 0.7) (layer "B.Cu") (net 15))
 (segment (start 134.075 65.5) (end 107.545989 65.5) (width 0.7) (layer "B.Cu") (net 15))
 (segment (start 147.2 115.7) (end 143.5 112) (width 0.7) (layer "F.Cu") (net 10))
 (segment (start 143.5 112) (end 123.2 112) (width 0.7) (layer "F.Cu") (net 10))
 (segment (start 123.2 112) (end 111.6 100.4) (width 0.7) (layer "F.Cu") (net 10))
 (segment (start 111.6 100.4) (end 99.2 100.4) (width 0.7) (layer "F.Cu") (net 10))
 (via (at 99.2 100.4) (size 1) (drill 0.5) (layers "F.Cu" "B.Cu") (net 10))
 (via (at 147.2 115.7) (size 1) (drill 0.5) (layers "F.Cu" "B.Cu") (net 10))
 (segment (start 95.6 96.8) (end 99.2 100.4) (width 0.7) (layer "B.Cu") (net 10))
 (segment (start 147.2 115.7) (end 147.2 117.875) (width 0.7) (layer "B.Cu") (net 10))
 (segment (start 98.5 88.5) (end 96.5 88.5) (width 0.7) (layer "B.Cu") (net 10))
 (segment (start 96.5 88.5) (end 95.6 89.4) (width 0.7) (layer "B.Cu") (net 10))
 (segment (start 95.6 89.4) (end 95.6 96.8) (width 0.7) (layer "B.Cu") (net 10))
 (segment (start 137.4 113.7) (end 122.5 113.7) (width 0.7) (layer "F.Cu") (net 11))
 (segment (start 139.4 115.7) (end 137.4 113.7) (width 0.7) (layer "F.Cu") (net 11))
 (segment (start 122.5 113.7) (end 111 102.2) (width 0.7) (layer "F.Cu") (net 11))
 (segment (start 111 102.2) (end 99.2 102.2) (width 0.7) (layer "F.Cu") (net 11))
 (via (at 139.4 115.7) (size 1) (drill 0.5) (layers "F.Cu" "B.Cu") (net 11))
 (via (at 99.2 102.2) (size 1) (drill 0.5) (layers "F.Cu" "B.Cu") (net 11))
 (segment (start 98.36 86.1) (end 96.8 86.1) (width 0.7) (layer "B.Cu") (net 11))
 (segment (start 139.4 115.7) (end 139.7 116) (width 0.7) (layer "B.Cu") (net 11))
 (segment (start 139.7 116) (end 139.7 117.875) (width 0.7) (layer "B.Cu") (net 11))
 (segment (start 96.8 86.1) (end 94.5 88.4) (width 0.7) (layer "B.Cu") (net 11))
 (segment (start 94.5 88.4) (end 94.5 97.5) (width 0.7) (layer "B.Cu") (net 11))
 (segment (start 94.5 97.5) (end 99.2 102.2) (width 0.7) (layer "B.Cu") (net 11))
 (segment (start 98.5 85.96) (end 98.36 86.1) (width 0.7) (layer "B.Cu") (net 11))
 (segment (start 95.8 76.3) (end 97.84 78.34) (width 0.7) (layer "B.Cu") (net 14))
 (segment (start 139.325 62.5) (end 108.990355 62.5) (width 0.7) (layer "B.Cu") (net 14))
 (segment (start 100.930355 70.56) (end 97.381623 70.56) (width 0.7) (layer "B.Cu") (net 14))
 (segment (start 97.381623 70.56) (end 95.8 72.141623) (width 0.7) (layer "B.Cu") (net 14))
 (segment (start 95.8 72.141623) (end 95.8 76.3) (width 0.7) (layer "B.Cu") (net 14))
 (segment (start 108.990355 62.5) (end 100.930355 70.56) (width 0.7) (layer "B.Cu") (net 14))
 (segment (start 97.84 78.34) (end 98.5 78.34) (width 0.7) (layer "B.Cu") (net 14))
 (segment (start 148 71.175) (end 139.325 62.5) (width 0.7) (layer "B.Cu") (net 14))
 (segment (start 155 71.1) (end 143.4 59.5) (width 0.7) (layer "B.Cu") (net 13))
 (segment (start 100.474721 69.46) (end 96.925988 69.46) (width 0.7) (layer "B.Cu") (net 13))
 (segment (start 143.4 59.5) (end 110.434721 59.5) (width 0.7) (layer "B.Cu") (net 13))
 (segment (start 98.18 80.88) (end 98.5 80.88) (width 0.7) (layer "B.Cu") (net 13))
 (segment (start 96.925988 69.46) (end 94.7 71.685988) (width 0.7) (layer "B.Cu") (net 13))
 (segment (start 110.434721 59.5) (end 100.474721 69.46) (width 0.7) (layer "B.Cu") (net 13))
 (segment (start 94.7 77.4) (end 98.18 80.88) (width 0.7) (layer "B.Cu") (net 13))
 (segment (start 94.7 71.685988) (end 94.7 77.4) (width 0.7) (layer "B.Cu") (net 13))
 (segment (start 123.8 110.4) (end 112 98.6) (width 0.7) (layer "F.Cu") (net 9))
 (segment (start 112 98.6) (end 99.5 98.6) (width 0.7) (layer "F.Cu") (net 9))
 (segment (start 149.5 110.4) (end 123.8 110.4) (width 0.7) (layer "F.Cu") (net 9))
 (segment (start 154.8 115.7) (end 149.5 110.4) (width 0.7) (layer "F.Cu") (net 9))
 (via (at 154.8 115.7) (size 1) (drill 0.5) (layers "F.Cu" "B.Cu") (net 9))
 (via (at 99.5 98.6) (size 1) (drill 0.5) (layers "F.Cu" "B.Cu") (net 9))
 (segment (start 98.5 91.04) (end 98.5 97.6) (width 0.7) (layer "B.Cu") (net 9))
 (segment (start 155 115.9) (end 155 117.875) (width 0.7) (layer "B.Cu") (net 9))
 (segment (start 154.8 115.7) (end 155 115.9) (width 0.7) (layer "B.Cu") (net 9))
 (segment (start 98.5 97.6) (end 99.5 98.6) (width 0.7) (layer "B.Cu") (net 9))
 (segment (start 110.5 103.8) (end 99.4 103.8) (width 0.7) (layer "F.Cu") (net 12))
 (segment (start 131.7 115.7) (end 131 115) (width 0.7) (layer "F.Cu") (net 12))
 (segment (start 121.7 115) (end 110.5 103.8) (width 0.7) (layer "F.Cu") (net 12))
 (segment (start 131 115) (end 121.7 115) (width 0.7) (layer "F.Cu") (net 12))
 (via (at 131.7 115.7) (size 1) (drill 0.5) (layers "F.Cu" "B.Cu") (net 12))
 (via (at 99.4 103.8) (size 1) (drill 0.5) (layers "F.Cu" "B.Cu") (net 12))
 (segment (start 99.4 103.8) (end 98.7 103.8) (width 0.7) (layer "B.Cu") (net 12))
 (segment (start 96.93 83.42) (end 98.5 83.42) (width 0.7) (layer "B.Cu") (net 12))
 (segment (start 98.7 103.8) (end 93.3 98.4) (width 0.7) (layer "B.Cu") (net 12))
 (segment (start 93.3 87.05) (end 96.93 83.42) (width 0.7) (layer "B.Cu") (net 12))
 (segment (start 93.3 98.4) (end 93.3 87.05) (width 0.7) (layer "B.Cu") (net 12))
 (segment (start 132.1 116.1) (end 132.1 117.875) (width 0.7) (layer "B.Cu") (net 12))
 (segment (start 131.7 115.7) (end 132.1 116.1) (width 0.7) (layer "B.Cu") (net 12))
 (segment (start 134 70.75) (end 134 68.9) (width 0.7) (layer "F.Cu") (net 16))
 (segment (start 134 68.9) (end 132.55 67.45) (width 0.7) (layer "F.Cu") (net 16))
 (via (at 134 70.75) (size 1) (drill 0.5) (layers "F.Cu" "B.Cu") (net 16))
 (via (at 132.55 67.45) (size 1) (drill 0.5) (layers "F.Cu" "B.Cu") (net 16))
 (segment (start 107.601624 67) (end 101.101624 73.5) (width 0.7) (layer "B.Cu") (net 16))
 (segment (start 134 70.75) (end 133.575 71.175) (width 0.7) (layer "B.Cu") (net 16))
 (segment (start 101.101624 73.5) (end 98.74 73.5) (width 0.7) (layer "B.Cu") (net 16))
 (segment (start 133.575 71.175) (end 132.5 71.175) (width 0.7) (layer "B.Cu") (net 16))
 (segment (start 98.74 73.5) (end 98.5 73.26) (width 0.7) (layer "B.Cu") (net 16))
 (segment (start 132.55 67.45) (end 132.1 67) (width 0.7) (layer "B.Cu") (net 16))
 (segment (start 132.1 67) (end 107.601624 67) (width 0.7) (layer "B.Cu") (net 16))
 (segment (start 148 74.88) (end 147.38 75.5) (width 0.7) (layer "B.Cu") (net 27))
 (segment (start 148 72.825) (end 148 74.88) (width 0.7) (layer "B.Cu") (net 27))
 (segment (start 147.2 122.12) (end 147.38 122.3) (width 0.7) (layer "B.Cu") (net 38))
 (segment (start 147.2 119.525) (end 147.2 122.12) (width 0.7) (layer "B.Cu") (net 38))
 (segment (start 139.75 75.49) (end 139.76 75.5) (width 0.7) (layer "B.Cu") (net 29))
 (segment (start 139.75 72.825) (end 139.75 75.49) (width 0.7) (layer "B.Cu") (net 29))
 (segment (start 152.25 75.29) (end 152.46 75.5) (width 0.7) (layer "B.Cu") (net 26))
 (segment (start 152.25 72.825) (end 152.25 75.29) (width 0.7) (layer "B.Cu") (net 26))
 (segment (start 136.75 72.825) (end 136.75 75.03) (width 0.7) (layer "B.Cu") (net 30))
 (segment (start 136.75 75.03) (end 137.22 75.5) (width 0.7) (layer "B.Cu") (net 30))
 (segment (start 144.4 119.525) (end 144.4 121.86) (width 0.7) (layer "B.Cu") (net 37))
 (segment (start 144.4 121.86) (end 144.84 122.3) (width 0.7) (layer "B.Cu") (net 37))
 (segment (start 145 75.34) (end 144.84 75.5) (width 0.7) (layer "B.Cu") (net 28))
 (segment (start 145 72.825) (end 145 75.34) (width 0.7) (layer "B.Cu") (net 28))
 (segment (start 132.1 119.525) (end 132.1 122.26) (width 0.7) (layer "B.Cu") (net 34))
 (segment (start 132.1 122.26) (end 132.14 122.3) (width 0.7) (layer "B.Cu") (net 34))
 (segment (start 136.9 119.525) (end 136.9 121.98) (width 0.7) (layer "B.Cu") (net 35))
 (segment (start 136.9 121.98) (end 137.22 122.3) (width 0.7) (layer "B.Cu") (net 35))
 (segment (start 129.5 119.525) (end 129.5 122.2) (width 0.7) (layer "B.Cu") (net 33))
 (segment (start 129.5 122.2) (end 129.6 122.3) (width 0.7) (layer "B.Cu") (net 33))
 (segment (start 155 72.75) (end 155 75.5) (width 0.7) (layer "B.Cu") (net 25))
 (segment (start 139.7 119.525) (end 139.7 122.24) (width 0.7) (layer "B.Cu") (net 36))
 (segment (start 139.7 122.24) (end 139.76 122.3) (width 0.7) (layer "B.Cu") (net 36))
 (segment (start 129.5 72.825) (end 129.5 75.4) (width 0.7) (layer "B.Cu") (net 32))
 (segment (start 129.5 75.4) (end 129.6 75.5) (width 0.7) (layer "B.Cu") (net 32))
 (segment (start 132.5 75.14) (end 132.14 75.5) (width 0.7) (layer "B.Cu") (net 31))
 (segment (start 132.5 72.825) (end 132.5 75.14) (width 0.7) (layer "B.Cu") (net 31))
 (segment (start 155 119.525) (end 155 122.3) (width 0.7) (layer "B.Cu") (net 40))
 (segment (start 151.9 119.525) (end 151.9 121.74) (width 0.7) (layer "B.Cu") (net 39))
 (segment (start 151.9 121.74) (end 152.46 122.3) (width 0.7) (layer "B.Cu") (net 39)))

